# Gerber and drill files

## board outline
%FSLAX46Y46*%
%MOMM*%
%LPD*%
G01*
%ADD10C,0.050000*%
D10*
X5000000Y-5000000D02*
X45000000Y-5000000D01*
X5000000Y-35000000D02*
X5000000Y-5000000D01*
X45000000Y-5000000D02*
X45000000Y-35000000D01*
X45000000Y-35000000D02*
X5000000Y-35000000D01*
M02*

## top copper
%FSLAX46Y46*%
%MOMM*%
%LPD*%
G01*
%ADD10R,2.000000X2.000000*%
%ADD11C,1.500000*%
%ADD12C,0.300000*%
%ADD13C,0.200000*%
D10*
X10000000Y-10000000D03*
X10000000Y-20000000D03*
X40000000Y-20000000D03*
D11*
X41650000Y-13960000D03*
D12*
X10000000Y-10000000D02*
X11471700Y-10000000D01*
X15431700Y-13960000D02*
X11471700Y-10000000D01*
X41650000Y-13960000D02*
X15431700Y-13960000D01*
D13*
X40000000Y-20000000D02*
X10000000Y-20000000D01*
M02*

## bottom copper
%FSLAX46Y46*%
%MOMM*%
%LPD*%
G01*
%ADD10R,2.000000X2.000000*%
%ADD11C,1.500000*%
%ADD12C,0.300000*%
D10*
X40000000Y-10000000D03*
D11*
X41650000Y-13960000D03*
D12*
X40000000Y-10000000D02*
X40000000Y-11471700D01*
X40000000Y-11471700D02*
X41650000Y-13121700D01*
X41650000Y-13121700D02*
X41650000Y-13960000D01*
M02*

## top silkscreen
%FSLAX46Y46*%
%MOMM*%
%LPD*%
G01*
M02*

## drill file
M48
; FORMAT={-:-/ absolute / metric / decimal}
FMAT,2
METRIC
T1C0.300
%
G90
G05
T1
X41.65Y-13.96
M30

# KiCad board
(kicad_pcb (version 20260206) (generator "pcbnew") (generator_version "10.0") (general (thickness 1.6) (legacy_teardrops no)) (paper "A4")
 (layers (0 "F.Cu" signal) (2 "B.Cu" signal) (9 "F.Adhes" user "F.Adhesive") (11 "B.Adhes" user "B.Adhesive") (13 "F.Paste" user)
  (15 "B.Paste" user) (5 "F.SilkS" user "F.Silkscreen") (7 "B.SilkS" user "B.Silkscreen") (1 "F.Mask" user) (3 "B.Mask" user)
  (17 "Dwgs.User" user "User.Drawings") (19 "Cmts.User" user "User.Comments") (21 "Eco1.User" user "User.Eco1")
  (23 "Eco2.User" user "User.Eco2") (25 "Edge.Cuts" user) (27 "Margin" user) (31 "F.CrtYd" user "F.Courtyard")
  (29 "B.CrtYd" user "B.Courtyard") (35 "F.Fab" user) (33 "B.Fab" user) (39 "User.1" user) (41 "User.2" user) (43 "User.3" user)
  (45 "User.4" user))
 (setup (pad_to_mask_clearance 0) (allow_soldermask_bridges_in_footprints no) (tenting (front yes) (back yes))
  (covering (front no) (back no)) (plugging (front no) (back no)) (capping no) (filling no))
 (gr_line (start 5 5) (end 45 5) (stroke (width 0.05) (type default)) (layer "Edge.Cuts"))
 (gr_line (start 5 35) (end 5 5) (stroke (width 0.05) (type default)) (layer "Edge.Cuts"))
 (gr_line (start 45 5) (end 45 35) (stroke (width 0.05) (type default)) (layer "Edge.Cuts"))
 (gr_line (start 45 35) (end 5 35) (stroke (width 0.05) (type default)) (layer "Edge.Cuts"))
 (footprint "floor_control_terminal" (layer "F.Cu") (at 10 10)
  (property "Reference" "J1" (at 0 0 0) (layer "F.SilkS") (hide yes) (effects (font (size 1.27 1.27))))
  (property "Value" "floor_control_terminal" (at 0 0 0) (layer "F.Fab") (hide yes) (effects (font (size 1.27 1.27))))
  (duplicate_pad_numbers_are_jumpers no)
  (pad "1" smd rect (at 0 0) (size 2 2) (layers "F.Cu" "F.Paste" "F.Mask") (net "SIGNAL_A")))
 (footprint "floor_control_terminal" (layer "B.Cu") (at 40 10)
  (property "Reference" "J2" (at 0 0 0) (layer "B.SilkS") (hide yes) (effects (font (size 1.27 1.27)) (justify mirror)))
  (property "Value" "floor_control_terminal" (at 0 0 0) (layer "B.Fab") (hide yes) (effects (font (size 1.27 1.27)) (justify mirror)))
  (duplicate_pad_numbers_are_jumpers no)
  (pad "1" smd rect (at 0 0) (size 2 2) (layers "B.Cu" "B.Paste" "B.Mask") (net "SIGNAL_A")))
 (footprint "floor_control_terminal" (layer "F.Cu") (at 10 20)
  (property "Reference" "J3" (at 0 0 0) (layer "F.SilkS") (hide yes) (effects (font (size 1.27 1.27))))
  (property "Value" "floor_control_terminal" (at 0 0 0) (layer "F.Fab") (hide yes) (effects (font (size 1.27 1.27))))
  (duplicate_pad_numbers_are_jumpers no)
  (pad "1" smd rect (at 0 0) (size 2 2) (layers "F.Cu" "F.Paste" "F.Mask") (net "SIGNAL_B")))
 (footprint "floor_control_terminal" (layer "F.Cu") (at 40 20)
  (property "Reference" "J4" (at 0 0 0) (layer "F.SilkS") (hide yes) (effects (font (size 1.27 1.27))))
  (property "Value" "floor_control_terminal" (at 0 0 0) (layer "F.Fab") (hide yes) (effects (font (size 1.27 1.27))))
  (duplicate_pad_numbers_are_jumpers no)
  (pad "1" smd rect (at 0 0) (size 2 2) (layers "F.Cu" "F.Paste" "F.Mask") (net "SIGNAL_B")))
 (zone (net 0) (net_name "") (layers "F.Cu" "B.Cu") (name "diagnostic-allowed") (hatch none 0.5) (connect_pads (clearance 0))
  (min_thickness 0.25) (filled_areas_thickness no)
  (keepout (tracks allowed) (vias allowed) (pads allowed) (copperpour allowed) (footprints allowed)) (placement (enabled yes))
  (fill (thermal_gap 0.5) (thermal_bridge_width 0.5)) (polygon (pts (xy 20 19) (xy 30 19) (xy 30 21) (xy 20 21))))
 (segment (start 10 10) (end 11.4717 10) (width 0.3) (layer "F.Cu") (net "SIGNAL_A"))
 (segment (start 15.4317 13.96) (end 11.4717 10) (width 0.3) (layer "F.Cu") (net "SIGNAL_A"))
 (segment (start 41.65 13.96) (end 15.4317 13.96) (width 0.3) (layer "F.Cu") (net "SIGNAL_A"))
 (via (at 41.65 13.96) (size 1.5) (drill 0.3) (layers "F.Cu" "B.Cu") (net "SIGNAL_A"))
 (segment (start 40 10) (end 40 11.4717) (width 0.3) (layer "B.Cu") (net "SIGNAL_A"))
 (segment (start 40 11.4717) (end 41.65 13.1217) (width 0.3) (layer "B.Cu") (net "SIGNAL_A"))
 (segment (start 41.65 13.1217) (end 41.65 13.96) (width 0.3) (layer "B.Cu") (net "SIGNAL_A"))
 (segment (start 40 20) (end 10 20) (width 0.2) (layer "F.Cu") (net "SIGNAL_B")))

